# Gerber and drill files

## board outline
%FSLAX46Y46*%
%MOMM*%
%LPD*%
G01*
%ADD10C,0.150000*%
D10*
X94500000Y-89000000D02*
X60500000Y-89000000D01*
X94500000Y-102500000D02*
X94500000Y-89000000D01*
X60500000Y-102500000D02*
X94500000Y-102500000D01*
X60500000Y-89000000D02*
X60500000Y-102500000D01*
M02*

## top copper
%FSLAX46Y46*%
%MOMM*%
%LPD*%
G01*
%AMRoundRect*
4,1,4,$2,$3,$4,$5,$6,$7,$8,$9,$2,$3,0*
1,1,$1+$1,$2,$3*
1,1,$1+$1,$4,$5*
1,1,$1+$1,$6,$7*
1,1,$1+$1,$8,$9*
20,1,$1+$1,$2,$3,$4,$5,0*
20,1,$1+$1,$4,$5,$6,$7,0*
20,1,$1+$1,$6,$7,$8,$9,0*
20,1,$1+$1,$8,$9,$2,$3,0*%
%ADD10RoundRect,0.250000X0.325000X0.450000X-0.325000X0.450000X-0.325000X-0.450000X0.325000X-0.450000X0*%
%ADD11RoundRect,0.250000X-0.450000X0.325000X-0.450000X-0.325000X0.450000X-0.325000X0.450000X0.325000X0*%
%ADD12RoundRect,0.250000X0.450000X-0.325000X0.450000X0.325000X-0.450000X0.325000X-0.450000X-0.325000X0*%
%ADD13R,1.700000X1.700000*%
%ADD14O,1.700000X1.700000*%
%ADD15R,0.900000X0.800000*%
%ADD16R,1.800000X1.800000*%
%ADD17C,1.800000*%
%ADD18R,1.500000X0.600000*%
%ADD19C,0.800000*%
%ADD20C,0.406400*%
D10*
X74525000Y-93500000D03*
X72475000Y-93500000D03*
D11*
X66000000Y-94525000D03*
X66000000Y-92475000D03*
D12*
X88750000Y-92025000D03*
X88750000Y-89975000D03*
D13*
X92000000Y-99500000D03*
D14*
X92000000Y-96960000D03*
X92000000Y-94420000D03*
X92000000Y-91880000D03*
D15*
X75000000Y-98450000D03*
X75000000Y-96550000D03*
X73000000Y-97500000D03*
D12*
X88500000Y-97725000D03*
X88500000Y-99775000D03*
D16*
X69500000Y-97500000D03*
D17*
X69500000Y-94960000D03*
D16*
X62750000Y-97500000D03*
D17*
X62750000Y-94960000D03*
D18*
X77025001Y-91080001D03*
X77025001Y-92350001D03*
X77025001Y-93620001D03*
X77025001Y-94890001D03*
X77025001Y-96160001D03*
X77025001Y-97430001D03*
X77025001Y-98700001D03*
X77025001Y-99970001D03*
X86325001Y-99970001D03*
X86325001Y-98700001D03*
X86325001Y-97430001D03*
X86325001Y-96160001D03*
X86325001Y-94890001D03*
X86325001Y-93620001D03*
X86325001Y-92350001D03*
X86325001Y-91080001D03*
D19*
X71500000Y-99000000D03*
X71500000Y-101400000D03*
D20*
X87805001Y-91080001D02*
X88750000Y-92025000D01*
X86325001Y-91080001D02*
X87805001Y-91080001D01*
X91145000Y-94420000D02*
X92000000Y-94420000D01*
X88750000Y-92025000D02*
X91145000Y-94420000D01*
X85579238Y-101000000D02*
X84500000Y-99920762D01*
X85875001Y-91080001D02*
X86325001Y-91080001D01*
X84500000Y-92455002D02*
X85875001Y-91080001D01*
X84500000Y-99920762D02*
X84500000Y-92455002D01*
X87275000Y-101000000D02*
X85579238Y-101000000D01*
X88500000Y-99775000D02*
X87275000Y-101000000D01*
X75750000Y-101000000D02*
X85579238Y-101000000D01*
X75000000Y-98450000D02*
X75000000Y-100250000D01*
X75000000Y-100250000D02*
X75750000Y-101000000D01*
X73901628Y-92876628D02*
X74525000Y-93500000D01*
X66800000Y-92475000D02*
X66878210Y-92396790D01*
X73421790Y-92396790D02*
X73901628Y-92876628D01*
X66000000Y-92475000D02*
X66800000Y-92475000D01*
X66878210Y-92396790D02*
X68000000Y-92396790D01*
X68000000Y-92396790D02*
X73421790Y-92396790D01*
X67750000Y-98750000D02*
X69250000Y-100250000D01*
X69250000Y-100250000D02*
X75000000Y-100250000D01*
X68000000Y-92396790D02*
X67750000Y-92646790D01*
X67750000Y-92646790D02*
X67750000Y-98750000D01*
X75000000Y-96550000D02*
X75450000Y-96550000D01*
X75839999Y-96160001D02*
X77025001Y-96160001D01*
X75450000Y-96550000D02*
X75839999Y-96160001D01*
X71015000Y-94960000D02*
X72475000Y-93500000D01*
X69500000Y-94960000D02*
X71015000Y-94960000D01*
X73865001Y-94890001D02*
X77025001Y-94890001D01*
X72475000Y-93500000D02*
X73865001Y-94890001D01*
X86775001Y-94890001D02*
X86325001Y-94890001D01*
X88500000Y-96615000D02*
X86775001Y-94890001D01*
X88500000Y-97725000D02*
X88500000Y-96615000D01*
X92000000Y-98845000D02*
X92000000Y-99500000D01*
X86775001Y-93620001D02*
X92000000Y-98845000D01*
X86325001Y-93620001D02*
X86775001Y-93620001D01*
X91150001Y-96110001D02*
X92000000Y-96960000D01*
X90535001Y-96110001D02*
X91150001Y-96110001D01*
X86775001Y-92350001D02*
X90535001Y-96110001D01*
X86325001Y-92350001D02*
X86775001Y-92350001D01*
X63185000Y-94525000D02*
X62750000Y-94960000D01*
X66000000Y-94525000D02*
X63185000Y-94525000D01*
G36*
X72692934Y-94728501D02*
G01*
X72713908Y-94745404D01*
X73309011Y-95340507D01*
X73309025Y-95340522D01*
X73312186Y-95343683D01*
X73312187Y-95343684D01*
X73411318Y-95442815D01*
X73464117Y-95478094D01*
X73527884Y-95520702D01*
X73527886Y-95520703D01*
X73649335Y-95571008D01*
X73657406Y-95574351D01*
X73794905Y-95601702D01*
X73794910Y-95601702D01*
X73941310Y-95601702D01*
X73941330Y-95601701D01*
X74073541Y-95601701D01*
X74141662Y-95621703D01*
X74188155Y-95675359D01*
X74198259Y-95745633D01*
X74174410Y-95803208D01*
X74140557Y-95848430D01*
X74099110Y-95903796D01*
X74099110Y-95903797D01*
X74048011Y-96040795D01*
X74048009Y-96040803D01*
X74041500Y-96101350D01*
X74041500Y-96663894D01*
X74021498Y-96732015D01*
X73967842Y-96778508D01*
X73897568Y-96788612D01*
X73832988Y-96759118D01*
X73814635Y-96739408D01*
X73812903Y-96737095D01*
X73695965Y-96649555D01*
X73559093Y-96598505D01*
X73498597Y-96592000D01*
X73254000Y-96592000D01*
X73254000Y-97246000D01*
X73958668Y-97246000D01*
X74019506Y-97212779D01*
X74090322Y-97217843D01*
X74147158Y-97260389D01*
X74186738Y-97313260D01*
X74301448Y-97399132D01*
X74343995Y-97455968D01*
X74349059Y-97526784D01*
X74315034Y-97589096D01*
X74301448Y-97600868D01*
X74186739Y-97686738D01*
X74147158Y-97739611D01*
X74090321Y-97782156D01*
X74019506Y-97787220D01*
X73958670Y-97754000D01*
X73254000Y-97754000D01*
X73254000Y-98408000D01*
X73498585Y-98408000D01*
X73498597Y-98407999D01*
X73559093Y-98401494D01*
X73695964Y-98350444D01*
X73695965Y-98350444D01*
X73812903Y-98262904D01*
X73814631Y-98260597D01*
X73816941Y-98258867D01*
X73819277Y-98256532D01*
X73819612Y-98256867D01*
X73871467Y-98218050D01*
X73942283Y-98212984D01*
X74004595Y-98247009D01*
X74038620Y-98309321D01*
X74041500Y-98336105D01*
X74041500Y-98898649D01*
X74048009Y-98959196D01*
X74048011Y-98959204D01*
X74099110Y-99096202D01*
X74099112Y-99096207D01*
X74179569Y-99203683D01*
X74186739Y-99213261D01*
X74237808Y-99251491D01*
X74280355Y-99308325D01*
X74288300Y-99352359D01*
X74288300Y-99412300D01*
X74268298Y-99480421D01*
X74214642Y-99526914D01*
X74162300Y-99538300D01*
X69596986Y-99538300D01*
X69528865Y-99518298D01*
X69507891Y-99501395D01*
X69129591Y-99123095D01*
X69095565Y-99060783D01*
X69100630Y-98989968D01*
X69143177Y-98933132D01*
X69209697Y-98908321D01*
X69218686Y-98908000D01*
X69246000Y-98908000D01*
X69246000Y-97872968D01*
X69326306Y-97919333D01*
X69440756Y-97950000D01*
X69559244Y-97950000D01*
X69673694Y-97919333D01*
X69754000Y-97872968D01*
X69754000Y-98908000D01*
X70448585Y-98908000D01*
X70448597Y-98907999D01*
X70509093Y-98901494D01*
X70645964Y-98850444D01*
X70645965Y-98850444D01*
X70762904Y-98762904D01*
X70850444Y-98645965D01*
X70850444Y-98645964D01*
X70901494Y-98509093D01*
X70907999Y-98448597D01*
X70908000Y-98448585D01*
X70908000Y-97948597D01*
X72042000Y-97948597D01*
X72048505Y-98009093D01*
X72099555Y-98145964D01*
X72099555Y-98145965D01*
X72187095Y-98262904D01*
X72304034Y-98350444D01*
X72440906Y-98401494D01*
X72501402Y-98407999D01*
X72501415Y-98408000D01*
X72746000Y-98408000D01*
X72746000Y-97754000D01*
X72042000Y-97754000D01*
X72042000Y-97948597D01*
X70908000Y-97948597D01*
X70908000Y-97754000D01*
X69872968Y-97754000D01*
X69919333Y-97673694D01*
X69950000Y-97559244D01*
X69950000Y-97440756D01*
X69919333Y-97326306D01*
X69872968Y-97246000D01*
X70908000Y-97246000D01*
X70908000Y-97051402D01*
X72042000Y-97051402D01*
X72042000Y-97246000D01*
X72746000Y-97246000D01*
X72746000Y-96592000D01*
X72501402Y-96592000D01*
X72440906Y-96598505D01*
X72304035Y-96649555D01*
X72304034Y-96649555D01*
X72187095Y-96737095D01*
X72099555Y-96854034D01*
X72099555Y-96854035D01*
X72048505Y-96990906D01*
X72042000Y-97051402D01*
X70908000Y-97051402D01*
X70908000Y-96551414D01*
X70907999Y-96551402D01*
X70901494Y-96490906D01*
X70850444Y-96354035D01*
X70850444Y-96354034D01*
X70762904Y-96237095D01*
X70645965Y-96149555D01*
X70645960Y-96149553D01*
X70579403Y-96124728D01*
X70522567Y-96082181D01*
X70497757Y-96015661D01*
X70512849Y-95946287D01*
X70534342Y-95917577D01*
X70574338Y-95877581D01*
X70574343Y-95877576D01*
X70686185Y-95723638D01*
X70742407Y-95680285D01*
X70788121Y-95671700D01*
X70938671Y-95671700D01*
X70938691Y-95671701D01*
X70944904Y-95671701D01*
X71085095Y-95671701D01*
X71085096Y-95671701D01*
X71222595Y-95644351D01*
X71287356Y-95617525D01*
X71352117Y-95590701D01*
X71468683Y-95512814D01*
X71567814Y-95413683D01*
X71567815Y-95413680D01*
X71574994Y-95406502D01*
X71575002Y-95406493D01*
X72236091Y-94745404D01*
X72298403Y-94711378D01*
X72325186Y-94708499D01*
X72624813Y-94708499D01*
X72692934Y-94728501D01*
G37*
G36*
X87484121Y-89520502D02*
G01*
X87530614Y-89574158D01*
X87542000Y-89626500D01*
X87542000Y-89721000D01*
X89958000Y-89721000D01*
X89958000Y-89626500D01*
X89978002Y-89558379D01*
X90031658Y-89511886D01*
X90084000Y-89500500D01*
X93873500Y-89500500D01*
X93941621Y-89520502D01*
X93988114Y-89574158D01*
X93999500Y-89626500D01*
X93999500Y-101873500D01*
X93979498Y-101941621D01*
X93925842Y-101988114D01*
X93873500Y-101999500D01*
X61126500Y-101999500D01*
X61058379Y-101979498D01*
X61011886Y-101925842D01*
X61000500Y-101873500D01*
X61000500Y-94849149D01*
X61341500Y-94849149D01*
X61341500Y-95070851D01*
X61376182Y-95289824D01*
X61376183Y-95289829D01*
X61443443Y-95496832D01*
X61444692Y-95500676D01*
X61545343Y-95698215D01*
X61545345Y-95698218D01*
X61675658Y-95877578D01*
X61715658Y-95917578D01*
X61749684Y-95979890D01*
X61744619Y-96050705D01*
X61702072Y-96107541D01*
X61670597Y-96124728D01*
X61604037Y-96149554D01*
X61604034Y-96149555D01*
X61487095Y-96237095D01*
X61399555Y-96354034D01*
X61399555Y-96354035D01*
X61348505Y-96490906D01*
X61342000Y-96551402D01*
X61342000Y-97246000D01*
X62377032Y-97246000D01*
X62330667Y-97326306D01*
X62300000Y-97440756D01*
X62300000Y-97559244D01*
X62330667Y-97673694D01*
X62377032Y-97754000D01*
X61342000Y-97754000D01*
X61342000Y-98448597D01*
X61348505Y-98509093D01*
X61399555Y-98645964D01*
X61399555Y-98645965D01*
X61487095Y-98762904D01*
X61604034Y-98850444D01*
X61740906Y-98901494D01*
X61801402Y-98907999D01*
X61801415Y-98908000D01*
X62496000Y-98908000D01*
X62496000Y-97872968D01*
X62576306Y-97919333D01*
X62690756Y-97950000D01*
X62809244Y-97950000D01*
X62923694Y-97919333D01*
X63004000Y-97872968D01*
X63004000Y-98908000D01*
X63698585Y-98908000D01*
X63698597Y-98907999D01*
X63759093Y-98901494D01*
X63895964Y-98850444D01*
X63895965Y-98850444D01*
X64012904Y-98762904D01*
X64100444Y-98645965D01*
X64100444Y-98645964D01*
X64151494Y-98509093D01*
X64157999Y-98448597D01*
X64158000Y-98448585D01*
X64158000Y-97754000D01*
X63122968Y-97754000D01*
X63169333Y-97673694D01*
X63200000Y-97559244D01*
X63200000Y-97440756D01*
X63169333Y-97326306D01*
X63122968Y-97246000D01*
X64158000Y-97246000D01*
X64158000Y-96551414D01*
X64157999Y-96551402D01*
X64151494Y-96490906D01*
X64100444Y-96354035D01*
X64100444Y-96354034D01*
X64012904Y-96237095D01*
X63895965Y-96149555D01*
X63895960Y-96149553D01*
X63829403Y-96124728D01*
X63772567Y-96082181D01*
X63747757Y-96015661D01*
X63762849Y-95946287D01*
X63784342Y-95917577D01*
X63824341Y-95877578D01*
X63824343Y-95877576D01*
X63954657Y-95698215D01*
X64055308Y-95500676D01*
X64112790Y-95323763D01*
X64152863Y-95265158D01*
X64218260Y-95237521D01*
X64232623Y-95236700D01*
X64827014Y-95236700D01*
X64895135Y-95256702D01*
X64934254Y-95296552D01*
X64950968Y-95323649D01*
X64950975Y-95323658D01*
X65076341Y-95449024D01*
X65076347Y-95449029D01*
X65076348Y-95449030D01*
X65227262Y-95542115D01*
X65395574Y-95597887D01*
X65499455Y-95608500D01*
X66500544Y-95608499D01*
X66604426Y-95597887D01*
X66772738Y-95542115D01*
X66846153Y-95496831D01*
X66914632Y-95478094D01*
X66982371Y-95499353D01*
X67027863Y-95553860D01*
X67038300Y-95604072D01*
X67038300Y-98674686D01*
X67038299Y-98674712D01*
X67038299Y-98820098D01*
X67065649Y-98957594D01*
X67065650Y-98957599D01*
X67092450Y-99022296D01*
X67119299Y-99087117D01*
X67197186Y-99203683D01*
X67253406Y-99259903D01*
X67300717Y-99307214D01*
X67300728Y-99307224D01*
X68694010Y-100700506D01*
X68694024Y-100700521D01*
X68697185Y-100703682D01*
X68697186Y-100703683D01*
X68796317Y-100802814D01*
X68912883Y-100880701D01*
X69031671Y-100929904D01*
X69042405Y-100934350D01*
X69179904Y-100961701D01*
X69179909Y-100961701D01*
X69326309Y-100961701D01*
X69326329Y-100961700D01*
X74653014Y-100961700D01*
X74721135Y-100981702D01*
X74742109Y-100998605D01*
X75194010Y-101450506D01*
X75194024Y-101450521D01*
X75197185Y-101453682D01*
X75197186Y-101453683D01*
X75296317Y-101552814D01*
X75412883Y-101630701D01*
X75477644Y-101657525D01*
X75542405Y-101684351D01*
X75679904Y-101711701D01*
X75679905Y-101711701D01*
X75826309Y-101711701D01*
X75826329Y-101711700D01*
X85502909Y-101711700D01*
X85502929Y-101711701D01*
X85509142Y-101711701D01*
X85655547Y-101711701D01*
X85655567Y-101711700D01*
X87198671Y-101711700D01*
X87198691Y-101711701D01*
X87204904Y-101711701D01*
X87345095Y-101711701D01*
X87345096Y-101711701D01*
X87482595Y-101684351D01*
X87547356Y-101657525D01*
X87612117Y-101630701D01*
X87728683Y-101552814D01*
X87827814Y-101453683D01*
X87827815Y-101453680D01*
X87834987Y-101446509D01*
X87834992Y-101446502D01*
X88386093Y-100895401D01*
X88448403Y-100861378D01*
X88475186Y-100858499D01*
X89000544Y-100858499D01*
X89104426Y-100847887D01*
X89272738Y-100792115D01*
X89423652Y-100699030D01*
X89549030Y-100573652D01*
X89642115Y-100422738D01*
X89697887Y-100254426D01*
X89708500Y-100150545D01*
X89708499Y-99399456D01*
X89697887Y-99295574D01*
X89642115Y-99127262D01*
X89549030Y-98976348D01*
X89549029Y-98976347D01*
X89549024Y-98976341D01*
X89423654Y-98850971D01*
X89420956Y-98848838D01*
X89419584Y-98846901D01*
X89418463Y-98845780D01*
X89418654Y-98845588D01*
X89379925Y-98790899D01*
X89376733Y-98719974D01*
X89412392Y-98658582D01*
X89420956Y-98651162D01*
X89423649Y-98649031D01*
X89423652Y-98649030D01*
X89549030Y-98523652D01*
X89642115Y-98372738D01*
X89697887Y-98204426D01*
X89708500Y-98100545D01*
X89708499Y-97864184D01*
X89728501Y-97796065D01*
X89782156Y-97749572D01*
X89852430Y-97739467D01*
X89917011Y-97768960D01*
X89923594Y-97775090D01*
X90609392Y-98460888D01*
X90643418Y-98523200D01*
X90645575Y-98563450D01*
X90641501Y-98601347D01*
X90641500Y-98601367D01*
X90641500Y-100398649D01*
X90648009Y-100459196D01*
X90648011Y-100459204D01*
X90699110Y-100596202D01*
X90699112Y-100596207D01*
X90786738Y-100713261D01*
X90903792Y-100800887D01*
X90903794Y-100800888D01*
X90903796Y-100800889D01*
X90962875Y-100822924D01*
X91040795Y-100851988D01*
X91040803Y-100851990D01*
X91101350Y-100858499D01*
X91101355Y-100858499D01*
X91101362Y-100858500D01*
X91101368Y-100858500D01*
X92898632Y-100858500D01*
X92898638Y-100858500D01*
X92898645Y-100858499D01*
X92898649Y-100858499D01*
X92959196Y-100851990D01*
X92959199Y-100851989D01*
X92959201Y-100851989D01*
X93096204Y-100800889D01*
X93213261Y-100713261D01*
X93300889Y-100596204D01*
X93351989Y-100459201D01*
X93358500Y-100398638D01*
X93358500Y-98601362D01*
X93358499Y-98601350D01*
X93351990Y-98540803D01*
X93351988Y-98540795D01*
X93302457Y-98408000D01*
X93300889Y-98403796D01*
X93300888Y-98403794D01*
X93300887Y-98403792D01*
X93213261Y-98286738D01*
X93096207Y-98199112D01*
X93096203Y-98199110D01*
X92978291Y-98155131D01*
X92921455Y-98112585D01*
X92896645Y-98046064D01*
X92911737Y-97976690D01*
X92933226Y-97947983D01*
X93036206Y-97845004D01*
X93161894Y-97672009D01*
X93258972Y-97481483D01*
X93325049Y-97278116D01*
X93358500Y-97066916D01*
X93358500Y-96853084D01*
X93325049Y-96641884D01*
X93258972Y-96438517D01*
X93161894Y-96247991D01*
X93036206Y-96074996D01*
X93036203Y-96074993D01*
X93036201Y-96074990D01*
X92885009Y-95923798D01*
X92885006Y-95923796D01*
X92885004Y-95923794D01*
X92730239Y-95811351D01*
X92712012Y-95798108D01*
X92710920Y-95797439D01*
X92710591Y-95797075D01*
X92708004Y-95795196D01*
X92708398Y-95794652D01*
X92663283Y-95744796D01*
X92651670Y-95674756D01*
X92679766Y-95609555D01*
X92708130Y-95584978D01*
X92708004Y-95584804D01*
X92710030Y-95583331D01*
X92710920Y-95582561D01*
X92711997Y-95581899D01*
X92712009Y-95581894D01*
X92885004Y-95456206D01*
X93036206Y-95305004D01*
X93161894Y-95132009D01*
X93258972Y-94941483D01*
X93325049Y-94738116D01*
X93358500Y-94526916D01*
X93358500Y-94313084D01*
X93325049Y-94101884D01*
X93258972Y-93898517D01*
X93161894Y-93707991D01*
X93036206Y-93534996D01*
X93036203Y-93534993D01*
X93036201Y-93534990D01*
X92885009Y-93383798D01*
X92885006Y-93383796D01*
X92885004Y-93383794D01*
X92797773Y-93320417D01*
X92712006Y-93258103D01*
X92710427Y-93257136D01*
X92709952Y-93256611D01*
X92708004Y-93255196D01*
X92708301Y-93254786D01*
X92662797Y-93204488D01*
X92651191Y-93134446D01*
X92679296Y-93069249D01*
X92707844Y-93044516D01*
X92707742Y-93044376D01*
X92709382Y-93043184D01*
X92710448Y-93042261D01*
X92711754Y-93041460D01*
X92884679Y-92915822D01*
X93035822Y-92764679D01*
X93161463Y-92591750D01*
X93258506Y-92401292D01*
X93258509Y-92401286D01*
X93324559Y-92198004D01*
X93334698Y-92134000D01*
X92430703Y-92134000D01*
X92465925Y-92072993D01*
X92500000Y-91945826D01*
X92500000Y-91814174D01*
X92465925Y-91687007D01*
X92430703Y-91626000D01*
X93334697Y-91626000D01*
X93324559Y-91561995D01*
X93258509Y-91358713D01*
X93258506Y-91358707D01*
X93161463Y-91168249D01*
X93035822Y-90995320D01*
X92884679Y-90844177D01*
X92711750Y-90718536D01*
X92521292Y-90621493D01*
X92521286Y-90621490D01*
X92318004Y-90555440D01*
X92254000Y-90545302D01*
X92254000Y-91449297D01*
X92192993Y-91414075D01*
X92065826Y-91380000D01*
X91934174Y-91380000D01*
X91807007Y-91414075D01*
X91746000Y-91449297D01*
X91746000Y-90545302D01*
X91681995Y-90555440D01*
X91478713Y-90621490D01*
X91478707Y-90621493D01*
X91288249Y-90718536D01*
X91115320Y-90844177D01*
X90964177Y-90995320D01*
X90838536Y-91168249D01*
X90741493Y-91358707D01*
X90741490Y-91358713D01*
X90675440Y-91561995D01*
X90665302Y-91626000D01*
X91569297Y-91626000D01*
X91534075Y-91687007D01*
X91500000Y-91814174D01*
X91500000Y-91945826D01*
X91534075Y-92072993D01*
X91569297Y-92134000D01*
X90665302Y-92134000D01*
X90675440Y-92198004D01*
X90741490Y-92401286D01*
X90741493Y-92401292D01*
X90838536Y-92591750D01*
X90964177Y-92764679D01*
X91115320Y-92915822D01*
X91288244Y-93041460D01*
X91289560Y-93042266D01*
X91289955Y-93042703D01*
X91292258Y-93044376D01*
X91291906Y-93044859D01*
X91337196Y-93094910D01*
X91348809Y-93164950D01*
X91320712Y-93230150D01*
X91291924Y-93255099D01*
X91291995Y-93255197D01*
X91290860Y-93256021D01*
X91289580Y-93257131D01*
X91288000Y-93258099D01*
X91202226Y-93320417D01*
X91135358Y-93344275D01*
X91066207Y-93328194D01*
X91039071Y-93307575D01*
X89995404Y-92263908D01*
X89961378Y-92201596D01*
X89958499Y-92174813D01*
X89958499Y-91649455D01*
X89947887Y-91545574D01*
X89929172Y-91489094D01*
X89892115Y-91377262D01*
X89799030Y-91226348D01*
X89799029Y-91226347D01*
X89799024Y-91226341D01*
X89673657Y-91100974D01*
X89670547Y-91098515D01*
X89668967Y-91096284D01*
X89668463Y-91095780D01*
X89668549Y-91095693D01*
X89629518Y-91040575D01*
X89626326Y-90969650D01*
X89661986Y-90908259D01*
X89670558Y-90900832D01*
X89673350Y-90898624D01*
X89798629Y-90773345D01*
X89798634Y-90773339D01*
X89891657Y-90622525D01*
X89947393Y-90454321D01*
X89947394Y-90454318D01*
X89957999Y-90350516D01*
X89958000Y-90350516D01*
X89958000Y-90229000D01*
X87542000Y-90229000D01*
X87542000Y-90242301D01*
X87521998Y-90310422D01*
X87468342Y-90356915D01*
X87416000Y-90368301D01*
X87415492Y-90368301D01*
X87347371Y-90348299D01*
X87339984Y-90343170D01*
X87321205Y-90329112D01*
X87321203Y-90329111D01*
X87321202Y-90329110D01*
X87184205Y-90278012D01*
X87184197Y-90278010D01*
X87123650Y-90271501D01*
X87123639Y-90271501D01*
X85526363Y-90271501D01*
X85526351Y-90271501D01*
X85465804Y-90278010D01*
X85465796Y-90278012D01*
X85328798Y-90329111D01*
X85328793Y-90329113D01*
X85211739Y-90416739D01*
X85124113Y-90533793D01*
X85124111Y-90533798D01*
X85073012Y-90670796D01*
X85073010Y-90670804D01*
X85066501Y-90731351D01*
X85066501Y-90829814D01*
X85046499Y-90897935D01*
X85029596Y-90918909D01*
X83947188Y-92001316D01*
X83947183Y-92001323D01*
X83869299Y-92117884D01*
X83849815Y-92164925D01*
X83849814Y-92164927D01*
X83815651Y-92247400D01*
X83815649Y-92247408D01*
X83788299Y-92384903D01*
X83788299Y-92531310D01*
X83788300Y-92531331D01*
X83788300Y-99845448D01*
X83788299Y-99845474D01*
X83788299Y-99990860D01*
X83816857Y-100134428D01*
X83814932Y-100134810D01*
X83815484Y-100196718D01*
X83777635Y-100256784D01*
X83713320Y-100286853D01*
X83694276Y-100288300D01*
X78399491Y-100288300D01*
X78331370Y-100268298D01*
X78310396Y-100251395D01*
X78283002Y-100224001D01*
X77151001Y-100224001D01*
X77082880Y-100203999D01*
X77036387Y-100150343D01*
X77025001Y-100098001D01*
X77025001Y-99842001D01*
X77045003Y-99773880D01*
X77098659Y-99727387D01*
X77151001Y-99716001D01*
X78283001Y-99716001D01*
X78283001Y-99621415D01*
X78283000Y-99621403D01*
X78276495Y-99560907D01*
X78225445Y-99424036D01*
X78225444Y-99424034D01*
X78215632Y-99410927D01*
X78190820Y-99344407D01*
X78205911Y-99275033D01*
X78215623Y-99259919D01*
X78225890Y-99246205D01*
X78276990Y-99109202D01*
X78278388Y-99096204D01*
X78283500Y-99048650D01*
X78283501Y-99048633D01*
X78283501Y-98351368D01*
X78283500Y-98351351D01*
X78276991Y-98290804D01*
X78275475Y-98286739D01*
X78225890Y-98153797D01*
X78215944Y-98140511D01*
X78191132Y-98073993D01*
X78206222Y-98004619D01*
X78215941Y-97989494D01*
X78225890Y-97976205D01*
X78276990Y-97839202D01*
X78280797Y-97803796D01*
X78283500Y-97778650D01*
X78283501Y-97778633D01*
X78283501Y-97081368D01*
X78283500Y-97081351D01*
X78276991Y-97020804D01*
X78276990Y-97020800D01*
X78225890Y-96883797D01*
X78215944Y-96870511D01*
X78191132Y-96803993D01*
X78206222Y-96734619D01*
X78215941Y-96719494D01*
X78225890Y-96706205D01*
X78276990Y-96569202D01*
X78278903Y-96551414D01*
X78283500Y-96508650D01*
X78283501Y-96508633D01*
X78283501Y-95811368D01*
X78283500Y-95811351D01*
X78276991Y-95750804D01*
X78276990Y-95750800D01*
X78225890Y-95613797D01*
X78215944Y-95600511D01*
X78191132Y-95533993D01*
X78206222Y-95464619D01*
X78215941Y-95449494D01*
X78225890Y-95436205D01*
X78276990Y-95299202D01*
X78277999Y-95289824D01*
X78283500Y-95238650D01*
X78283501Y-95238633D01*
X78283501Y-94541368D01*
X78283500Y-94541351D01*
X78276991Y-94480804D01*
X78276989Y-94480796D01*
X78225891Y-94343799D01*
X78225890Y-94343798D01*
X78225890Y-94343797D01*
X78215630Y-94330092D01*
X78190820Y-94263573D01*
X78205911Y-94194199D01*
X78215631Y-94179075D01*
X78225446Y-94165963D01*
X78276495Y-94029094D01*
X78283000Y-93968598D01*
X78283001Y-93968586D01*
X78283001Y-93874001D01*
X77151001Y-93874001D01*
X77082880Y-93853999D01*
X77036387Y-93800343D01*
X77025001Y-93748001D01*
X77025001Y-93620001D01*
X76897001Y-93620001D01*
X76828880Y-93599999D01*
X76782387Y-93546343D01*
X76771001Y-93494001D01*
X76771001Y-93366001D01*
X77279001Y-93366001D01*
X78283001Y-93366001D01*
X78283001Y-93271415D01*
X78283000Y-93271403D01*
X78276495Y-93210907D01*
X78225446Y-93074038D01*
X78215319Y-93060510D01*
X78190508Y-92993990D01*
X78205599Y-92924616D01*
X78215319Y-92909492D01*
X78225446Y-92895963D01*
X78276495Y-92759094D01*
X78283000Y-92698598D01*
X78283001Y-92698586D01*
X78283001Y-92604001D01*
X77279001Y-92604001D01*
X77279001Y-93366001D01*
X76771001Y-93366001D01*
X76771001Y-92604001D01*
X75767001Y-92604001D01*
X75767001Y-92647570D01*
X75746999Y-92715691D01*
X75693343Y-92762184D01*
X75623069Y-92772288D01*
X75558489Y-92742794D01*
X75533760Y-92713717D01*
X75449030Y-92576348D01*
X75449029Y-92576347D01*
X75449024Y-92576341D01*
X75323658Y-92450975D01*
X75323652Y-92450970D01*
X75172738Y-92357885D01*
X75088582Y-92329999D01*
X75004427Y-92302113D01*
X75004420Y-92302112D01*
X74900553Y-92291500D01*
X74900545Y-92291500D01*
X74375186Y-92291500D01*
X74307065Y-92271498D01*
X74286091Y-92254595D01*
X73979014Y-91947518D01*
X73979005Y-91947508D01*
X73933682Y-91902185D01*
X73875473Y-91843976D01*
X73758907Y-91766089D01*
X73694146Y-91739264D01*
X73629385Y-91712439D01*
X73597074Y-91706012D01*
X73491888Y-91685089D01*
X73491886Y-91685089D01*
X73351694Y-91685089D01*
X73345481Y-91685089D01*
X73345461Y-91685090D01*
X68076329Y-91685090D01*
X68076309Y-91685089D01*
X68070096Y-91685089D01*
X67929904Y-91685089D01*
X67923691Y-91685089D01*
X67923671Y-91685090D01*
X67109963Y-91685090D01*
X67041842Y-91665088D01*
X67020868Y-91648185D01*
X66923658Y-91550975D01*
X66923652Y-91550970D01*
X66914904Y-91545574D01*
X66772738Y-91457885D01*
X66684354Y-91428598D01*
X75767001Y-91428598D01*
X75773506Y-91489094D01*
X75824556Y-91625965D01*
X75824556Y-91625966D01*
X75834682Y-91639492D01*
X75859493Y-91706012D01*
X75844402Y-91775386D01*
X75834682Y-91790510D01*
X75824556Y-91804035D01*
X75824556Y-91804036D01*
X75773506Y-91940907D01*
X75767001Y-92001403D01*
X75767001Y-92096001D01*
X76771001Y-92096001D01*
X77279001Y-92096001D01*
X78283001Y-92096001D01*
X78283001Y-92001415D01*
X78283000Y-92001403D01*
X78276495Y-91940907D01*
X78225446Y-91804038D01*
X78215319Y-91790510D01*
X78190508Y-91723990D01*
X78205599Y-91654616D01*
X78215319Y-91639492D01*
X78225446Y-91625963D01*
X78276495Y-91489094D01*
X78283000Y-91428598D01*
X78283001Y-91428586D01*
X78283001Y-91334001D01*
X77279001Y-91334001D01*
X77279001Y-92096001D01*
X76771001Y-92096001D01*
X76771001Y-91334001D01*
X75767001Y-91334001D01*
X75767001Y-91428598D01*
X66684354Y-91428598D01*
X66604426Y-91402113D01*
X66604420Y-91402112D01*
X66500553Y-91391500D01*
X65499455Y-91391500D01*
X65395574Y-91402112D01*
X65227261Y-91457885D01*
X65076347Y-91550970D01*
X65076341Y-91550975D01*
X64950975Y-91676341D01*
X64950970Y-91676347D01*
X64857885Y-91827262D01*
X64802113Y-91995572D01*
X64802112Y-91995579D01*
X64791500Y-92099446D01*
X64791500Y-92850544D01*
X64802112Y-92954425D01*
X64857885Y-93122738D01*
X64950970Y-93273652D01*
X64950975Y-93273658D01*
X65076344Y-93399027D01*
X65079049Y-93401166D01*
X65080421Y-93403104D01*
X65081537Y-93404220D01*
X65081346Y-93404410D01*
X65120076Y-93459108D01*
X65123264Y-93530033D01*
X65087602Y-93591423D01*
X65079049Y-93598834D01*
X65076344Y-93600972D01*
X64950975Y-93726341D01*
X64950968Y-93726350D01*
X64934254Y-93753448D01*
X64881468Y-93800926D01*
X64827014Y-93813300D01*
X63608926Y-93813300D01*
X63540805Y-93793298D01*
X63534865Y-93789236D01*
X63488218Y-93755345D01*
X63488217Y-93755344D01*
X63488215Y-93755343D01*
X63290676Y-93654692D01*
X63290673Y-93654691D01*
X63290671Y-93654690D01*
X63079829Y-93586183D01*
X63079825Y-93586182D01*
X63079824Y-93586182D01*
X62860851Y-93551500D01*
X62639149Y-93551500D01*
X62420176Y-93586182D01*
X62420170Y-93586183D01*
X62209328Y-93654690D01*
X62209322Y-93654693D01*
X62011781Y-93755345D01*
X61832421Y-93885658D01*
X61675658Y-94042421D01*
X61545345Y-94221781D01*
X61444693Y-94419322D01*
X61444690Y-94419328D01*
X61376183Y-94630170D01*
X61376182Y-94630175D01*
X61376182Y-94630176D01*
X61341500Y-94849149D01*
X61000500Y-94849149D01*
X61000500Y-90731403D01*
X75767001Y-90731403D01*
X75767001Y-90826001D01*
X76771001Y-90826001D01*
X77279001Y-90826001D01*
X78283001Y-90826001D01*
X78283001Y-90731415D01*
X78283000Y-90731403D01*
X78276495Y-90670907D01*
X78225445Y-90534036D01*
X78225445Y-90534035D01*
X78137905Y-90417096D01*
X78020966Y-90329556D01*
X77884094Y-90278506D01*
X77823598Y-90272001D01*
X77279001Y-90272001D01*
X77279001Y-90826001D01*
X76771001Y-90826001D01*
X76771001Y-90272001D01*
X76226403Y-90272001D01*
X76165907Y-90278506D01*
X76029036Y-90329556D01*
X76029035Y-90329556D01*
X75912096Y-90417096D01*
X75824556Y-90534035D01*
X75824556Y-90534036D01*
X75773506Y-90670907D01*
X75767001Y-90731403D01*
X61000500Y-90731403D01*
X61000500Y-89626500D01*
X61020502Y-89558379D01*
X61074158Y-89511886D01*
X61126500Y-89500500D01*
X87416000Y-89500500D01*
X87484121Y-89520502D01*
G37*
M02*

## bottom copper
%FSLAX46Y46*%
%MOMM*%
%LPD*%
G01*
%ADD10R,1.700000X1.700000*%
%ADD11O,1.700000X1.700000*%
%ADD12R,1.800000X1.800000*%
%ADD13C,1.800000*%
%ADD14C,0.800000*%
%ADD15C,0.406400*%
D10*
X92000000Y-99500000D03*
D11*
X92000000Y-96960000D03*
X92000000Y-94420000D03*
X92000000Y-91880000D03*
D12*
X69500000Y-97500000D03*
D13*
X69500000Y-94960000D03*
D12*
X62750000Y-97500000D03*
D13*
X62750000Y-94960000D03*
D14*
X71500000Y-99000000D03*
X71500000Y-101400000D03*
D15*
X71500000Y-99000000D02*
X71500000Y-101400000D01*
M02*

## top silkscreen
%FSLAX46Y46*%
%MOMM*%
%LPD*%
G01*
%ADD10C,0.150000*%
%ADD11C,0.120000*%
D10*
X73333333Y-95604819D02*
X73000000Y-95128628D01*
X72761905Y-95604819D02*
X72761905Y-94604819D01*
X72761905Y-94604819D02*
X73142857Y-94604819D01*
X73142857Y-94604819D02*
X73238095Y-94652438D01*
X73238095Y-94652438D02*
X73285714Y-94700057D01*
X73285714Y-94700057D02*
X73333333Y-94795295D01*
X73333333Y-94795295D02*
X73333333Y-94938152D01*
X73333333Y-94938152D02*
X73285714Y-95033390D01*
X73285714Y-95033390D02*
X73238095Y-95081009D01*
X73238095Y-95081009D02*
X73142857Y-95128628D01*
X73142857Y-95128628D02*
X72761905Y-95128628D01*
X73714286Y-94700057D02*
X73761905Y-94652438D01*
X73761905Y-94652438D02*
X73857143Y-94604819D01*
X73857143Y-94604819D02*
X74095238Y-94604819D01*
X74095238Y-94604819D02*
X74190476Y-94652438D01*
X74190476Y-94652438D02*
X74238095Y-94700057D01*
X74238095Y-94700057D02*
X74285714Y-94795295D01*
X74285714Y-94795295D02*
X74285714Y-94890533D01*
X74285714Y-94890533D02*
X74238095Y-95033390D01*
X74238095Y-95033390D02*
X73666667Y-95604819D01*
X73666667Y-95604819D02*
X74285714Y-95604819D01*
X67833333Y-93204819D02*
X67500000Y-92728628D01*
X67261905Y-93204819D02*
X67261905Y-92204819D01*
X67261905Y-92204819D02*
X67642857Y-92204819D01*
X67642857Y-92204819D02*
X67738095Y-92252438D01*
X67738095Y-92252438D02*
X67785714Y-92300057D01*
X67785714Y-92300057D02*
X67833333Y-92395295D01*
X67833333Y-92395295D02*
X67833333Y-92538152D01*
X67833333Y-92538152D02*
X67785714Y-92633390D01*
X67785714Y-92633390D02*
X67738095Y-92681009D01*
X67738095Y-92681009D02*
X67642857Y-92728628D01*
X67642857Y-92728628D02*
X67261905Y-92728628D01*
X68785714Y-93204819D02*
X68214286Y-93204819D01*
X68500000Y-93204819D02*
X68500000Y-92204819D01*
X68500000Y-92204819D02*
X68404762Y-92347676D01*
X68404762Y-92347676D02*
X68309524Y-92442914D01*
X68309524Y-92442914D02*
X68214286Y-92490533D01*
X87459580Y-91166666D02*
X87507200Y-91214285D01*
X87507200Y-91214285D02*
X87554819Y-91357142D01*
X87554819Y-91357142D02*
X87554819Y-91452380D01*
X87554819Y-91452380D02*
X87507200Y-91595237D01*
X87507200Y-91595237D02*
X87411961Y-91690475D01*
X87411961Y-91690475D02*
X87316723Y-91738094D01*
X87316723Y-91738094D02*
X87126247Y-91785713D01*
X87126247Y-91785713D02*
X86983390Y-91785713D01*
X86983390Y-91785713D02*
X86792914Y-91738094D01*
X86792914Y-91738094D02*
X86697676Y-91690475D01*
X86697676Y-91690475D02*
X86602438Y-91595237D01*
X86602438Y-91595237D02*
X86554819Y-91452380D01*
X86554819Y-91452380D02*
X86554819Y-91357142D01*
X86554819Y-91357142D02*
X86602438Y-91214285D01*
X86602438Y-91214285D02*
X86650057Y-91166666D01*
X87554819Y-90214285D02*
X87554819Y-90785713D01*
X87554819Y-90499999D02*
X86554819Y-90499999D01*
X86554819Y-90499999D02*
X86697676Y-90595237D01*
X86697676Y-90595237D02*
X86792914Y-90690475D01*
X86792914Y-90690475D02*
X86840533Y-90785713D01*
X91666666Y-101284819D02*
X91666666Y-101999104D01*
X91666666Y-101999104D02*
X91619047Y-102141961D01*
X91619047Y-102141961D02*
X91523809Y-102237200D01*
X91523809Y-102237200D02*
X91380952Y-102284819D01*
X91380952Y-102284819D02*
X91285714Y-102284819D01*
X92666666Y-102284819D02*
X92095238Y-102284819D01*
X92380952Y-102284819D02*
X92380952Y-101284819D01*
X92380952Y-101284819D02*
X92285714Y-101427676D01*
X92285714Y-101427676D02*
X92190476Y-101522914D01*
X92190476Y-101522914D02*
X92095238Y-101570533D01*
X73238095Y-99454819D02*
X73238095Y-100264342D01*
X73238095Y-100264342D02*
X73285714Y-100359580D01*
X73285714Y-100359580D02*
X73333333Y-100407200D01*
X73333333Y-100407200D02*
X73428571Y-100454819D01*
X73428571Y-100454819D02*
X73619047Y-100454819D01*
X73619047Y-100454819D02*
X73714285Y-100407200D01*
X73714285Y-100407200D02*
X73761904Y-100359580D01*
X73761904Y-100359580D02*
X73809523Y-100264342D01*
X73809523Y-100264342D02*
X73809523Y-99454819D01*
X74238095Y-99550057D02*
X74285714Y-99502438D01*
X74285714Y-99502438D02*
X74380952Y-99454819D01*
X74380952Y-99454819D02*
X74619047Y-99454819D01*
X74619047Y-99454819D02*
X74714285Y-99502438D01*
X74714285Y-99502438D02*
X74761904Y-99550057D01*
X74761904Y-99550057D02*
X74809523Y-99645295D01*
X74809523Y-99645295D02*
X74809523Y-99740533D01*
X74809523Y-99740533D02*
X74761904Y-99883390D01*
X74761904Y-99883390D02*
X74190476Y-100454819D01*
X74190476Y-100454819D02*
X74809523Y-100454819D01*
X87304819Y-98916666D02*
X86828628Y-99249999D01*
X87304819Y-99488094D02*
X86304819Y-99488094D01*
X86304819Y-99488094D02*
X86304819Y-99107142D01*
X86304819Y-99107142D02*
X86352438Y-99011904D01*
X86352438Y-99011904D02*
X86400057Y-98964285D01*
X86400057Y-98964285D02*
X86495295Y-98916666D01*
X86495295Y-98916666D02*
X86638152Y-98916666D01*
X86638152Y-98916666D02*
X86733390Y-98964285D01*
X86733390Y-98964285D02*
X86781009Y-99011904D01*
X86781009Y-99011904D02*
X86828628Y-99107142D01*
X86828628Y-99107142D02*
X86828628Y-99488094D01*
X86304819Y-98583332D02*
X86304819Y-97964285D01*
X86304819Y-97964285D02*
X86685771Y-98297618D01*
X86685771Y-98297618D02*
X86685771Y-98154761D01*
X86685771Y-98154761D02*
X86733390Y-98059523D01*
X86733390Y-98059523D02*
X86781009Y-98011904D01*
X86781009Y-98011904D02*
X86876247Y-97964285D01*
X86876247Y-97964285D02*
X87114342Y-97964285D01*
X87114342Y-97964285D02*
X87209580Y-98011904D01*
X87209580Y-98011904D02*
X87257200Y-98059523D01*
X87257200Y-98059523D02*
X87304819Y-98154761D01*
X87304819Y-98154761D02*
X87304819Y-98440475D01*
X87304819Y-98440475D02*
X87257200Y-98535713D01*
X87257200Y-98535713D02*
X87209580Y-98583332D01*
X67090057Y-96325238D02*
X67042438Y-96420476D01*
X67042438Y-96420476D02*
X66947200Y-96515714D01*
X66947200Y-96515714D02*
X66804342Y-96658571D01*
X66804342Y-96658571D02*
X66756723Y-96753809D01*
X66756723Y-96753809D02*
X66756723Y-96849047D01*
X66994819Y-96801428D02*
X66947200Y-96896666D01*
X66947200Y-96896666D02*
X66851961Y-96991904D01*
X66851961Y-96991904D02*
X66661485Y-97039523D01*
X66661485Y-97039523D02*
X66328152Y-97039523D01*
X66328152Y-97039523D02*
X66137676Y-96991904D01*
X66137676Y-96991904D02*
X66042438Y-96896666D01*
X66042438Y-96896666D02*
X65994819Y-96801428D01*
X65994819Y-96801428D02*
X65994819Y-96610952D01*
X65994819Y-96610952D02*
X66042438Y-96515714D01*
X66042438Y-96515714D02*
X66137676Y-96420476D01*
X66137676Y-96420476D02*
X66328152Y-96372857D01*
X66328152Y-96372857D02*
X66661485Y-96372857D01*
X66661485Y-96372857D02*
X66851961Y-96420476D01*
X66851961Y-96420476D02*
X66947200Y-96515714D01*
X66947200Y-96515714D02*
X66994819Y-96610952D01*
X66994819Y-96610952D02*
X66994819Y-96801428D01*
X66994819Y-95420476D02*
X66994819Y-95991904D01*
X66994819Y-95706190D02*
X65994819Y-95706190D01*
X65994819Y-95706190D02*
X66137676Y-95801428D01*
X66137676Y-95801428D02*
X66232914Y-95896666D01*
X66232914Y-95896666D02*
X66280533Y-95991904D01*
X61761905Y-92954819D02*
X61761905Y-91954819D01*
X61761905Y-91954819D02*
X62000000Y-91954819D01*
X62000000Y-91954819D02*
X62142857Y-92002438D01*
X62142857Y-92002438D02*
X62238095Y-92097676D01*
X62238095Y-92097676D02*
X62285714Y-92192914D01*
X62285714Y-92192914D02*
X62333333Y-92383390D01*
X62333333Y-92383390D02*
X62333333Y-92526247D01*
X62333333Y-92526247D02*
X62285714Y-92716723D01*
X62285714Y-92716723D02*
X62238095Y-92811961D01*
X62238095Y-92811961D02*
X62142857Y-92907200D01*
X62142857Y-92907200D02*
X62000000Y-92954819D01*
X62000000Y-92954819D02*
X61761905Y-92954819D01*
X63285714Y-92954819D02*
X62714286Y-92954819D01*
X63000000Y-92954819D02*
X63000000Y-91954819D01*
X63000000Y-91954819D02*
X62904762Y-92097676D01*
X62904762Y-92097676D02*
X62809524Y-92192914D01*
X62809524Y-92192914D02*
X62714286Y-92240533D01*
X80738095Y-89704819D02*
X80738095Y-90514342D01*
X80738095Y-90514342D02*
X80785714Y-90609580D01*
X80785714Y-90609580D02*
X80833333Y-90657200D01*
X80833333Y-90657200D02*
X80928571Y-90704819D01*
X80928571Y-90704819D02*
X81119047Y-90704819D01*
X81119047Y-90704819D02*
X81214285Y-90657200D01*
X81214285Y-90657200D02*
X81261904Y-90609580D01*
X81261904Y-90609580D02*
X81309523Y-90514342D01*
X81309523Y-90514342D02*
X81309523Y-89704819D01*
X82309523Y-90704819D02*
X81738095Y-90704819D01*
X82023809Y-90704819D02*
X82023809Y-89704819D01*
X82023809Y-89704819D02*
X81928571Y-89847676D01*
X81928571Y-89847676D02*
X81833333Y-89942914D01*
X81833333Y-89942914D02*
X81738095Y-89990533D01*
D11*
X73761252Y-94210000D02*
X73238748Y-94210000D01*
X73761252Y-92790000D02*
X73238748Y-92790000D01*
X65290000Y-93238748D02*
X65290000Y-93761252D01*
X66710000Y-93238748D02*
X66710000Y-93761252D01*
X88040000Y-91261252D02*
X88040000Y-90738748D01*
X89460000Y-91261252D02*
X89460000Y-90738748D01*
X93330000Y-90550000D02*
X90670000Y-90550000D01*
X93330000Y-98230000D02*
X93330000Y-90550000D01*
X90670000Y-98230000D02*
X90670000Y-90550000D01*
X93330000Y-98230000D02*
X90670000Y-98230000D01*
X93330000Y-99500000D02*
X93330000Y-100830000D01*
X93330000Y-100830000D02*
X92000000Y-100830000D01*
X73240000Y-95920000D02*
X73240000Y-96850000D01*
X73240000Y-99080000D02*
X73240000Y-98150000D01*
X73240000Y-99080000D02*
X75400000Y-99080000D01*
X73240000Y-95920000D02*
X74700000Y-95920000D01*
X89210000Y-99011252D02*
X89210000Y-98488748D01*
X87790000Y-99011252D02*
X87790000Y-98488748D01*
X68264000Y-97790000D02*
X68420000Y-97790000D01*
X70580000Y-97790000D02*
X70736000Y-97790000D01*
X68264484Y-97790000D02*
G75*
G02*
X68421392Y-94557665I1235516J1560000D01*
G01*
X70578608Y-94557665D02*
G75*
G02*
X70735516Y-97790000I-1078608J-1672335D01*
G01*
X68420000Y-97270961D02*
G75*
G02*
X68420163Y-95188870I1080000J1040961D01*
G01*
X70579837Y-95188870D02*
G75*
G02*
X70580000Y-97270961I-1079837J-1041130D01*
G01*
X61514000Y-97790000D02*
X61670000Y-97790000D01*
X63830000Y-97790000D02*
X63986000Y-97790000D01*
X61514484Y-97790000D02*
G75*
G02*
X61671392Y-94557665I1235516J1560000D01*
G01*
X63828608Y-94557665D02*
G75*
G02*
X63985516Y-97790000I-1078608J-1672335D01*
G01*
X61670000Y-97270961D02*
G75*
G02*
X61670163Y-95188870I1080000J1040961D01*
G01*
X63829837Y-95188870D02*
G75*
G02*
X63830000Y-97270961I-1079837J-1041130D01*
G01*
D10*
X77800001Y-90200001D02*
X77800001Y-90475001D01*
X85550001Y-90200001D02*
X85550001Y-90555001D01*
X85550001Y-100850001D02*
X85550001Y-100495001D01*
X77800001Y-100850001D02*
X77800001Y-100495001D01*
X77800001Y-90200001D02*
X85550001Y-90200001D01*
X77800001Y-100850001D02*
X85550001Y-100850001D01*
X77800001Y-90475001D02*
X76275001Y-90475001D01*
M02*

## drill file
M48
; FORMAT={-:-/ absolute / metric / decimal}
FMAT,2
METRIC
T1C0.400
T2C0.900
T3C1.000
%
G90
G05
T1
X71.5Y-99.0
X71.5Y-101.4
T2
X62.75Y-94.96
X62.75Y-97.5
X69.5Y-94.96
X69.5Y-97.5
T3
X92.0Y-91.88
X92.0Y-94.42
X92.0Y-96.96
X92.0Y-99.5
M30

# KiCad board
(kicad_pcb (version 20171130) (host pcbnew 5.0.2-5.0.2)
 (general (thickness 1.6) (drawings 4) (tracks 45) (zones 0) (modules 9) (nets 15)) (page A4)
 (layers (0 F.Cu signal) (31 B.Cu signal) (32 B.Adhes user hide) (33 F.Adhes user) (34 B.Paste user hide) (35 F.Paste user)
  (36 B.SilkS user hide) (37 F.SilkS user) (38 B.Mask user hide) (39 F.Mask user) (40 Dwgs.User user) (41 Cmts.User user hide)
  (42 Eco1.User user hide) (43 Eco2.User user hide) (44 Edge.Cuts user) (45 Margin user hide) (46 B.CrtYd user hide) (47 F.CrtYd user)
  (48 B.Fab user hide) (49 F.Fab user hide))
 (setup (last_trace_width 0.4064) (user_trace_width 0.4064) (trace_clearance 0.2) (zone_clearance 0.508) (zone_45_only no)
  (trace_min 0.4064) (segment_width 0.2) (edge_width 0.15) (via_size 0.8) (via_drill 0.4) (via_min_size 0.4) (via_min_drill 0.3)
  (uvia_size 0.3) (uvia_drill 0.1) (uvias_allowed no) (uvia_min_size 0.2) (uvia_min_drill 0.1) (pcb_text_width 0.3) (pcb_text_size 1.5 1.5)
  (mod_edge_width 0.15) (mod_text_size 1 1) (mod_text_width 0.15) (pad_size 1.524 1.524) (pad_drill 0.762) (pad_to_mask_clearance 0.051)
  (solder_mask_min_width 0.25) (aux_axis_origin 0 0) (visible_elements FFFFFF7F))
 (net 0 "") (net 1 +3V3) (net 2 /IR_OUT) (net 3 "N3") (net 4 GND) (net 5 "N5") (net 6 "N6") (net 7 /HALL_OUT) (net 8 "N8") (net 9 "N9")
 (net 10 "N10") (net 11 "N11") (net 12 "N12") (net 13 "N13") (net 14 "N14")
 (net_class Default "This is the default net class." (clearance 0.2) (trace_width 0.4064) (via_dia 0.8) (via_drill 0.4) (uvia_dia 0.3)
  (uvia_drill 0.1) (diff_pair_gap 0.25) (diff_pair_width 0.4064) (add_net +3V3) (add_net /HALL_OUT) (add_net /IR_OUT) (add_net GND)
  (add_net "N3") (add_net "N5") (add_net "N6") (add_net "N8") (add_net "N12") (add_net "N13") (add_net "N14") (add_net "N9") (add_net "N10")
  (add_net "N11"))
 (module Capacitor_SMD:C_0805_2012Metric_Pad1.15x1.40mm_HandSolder (layer F.Cu) (at 73.5 93.5 180)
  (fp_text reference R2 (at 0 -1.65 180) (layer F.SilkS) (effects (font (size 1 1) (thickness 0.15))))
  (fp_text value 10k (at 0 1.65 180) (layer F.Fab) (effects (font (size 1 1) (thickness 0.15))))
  (fp_line (start -0.261252 -0.71) (end 0.261252 -0.71) (layer F.SilkS) (width 0.12))
  (fp_line (start -0.261252 0.71) (end 0.261252 0.71) (layer F.SilkS) (width 0.12))
  (pad 1 smd roundrect (at -1.025 0 180) (size 1.15 1.4) (layers F.Cu F.Paste F.Mask) (roundrect_rratio 0.217391) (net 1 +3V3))
  (pad 2 smd roundrect (at 1.025 0 180) (size 1.15 1.4) (layers F.Cu F.Paste F.Mask) (roundrect_rratio 0.217391) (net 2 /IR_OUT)))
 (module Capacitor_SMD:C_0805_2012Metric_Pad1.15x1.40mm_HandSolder (layer F.Cu) (at 66 93.5 270)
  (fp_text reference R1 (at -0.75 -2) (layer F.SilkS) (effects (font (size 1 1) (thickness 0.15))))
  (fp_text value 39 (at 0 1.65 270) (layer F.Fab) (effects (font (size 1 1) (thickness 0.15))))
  (fp_line (start -0.261252 0.71) (end 0.261252 0.71) (layer F.SilkS) (width 0.12))
  (fp_line (start -0.261252 -0.71) (end 0.261252 -0.71) (layer F.SilkS) (width 0.12))
  (pad 2 smd roundrect (at 1.025 0 270) (size 1.15 1.4) (layers F.Cu F.Paste F.Mask) (roundrect_rratio 0.217391) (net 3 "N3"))
  (pad 1 smd roundrect (at -1.025 0 270) (size 1.15 1.4) (layers F.Cu F.Paste F.Mask) (roundrect_rratio 0.217391) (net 1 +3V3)))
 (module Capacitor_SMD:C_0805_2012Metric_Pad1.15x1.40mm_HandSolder (layer F.Cu) (at 88.75 91 90)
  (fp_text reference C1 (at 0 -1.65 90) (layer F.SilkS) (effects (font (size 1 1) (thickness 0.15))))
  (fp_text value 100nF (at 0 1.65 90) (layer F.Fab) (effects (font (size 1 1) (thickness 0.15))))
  (fp_line (start -0.261252 -0.71) (end 0.261252 -0.71) (layer F.SilkS) (width 0.12))
  (fp_line (start -0.261252 0.71) (end 0.261252 0.71) (layer F.SilkS) (width 0.12))
  (pad 1 smd roundrect (at -1.025 0 90) (size 1.15 1.4) (layers F.Cu F.Paste F.Mask) (roundrect_rratio 0.217391) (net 1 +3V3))
  (pad 2 smd roundrect (at 1.025 0 90) (size 1.15 1.4) (layers F.Cu F.Paste F.Mask) (roundrect_rratio 0.217391) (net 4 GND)))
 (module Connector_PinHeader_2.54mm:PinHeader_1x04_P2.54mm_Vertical (layer F.Cu) (at 92 99.5 180)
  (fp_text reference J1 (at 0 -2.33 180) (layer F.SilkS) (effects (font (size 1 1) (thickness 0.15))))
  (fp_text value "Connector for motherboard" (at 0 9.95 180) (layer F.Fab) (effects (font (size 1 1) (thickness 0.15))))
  (fp_line (start -1.33 8.95) (end 1.33 8.95) (layer F.SilkS) (width 0.12))
  (fp_line (start -1.33 1.27) (end -1.33 8.95) (layer F.SilkS) (width 0.12))
  (fp_line (start 1.33 1.27) (end 1.33 8.95) (layer F.SilkS) (width 0.12))
  (fp_line (start -1.33 1.27) (end 1.33 1.27) (layer F.SilkS) (width 0.12))
  (fp_line (start -1.33 0) (end -1.33 -1.33) (layer F.SilkS) (width 0.12))
  (fp_line (start -1.33 -1.33) (end 0 -1.33) (layer F.SilkS) (width 0.12))
  (pad 1 thru_hole rect (at 0 0 180) (size 1.7 1.7) (drill 1) (layers *.Cu *.Mask) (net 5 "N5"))
  (pad 2 thru_hole oval (at 0 2.54 180) (size 1.7 1.7) (drill 1) (layers *.Cu *.Mask) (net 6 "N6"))
  (pad 3 thru_hole oval (at 0 5.08 180) (size 1.7 1.7) (drill 1) (layers *.Cu *.Mask) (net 1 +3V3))
  (pad 4 thru_hole oval (at 0 7.62 180) (size 1.7 1.7) (drill 1) (layers *.Cu *.Mask) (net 4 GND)))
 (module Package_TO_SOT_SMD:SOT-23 (layer F.Cu) (at 74 97.5 180)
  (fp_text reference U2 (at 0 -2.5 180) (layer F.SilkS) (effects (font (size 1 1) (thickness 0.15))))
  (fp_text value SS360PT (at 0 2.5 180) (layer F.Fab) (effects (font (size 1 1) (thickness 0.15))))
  (fp_line (start 0.76 1.58) (end 0.76 0.65) (layer F.SilkS) (width 0.12))
  (fp_line (start 0.76 -1.58) (end 0.76 -0.65) (layer F.SilkS) (width 0.12))
  (fp_line (start 0.76 -1.58) (end -1.4 -1.58) (layer F.SilkS) (width 0.12))
  (fp_line (start 0.76 1.58) (end -0.7 1.58) (layer F.SilkS) (width 0.12))
  (pad 1 smd rect (at -1 -0.95 180) (size 0.9 0.8) (layers F.Cu F.Paste F.Mask) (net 1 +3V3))
  (pad 2 smd rect (at -1 0.95 180) (size 0.9 0.8) (layers F.Cu F.Paste F.Mask) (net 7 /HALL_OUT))
  (pad 3 smd rect (at 1 0 180) (size 0.9 0.8) (layers F.Cu F.Paste F.Mask) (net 4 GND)))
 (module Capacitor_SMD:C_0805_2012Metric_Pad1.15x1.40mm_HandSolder (layer F.Cu) (at 88.5 98.75 90)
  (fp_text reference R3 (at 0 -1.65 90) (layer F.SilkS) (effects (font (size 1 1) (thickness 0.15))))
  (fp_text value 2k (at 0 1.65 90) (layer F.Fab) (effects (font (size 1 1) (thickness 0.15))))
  (fp_line (start -0.261252 0.71) (end 0.261252 0.71) (layer F.SilkS) (width 0.12))
  (fp_line (start -0.261252 -0.71) (end 0.261252 -0.71) (layer F.SilkS) (width 0.12))
  (pad 2 smd roundrect (at 1.025 0 90) (size 1.15 1.4) (layers F.Cu F.Paste F.Mask) (roundrect_rratio 0.217391) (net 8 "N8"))
  (pad 1 smd roundrect (at -1.025 0 90) (size 1.15 1.4) (layers F.Cu F.Paste F.Mask) (roundrect_rratio 0.217391) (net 1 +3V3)))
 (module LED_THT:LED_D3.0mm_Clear (layer F.Cu) (at 69.5 97.5 90)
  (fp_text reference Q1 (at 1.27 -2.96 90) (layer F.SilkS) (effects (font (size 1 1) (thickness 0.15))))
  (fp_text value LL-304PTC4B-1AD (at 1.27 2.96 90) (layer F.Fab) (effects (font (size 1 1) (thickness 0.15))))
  (fp_line (start -0.29 -1.236) (end -0.29 -1.08) (layer F.SilkS) (width 0.12))
  (fp_line (start -0.29 1.08) (end -0.29 1.236) (layer F.SilkS) (width 0.12))
  (fp_arc (start 1.27 0) (end -0.29 -1.235516) (angle 108.8) (layer F.SilkS) (width 0.12))
  (fp_arc (start 1.27 0) (end -0.29 1.235516) (angle -108.8) (layer F.SilkS) (width 0.12))
  (fp_arc (start 1.27 0) (end 0.229039 -1.08) (angle 87.9) (layer F.SilkS) (width 0.12))
  (fp_arc (start 1.27 0) (end 0.229039 1.08) (angle -87.9) (layer F.SilkS) (width 0.12))
  (pad 1 thru_hole rect (at 0 0 90) (size 1.8 1.8) (drill 0.9) (layers *.Cu *.Mask) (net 4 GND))
  (pad 2 thru_hole circle (at 2.54 0 90) (size 1.8 1.8) (drill 0.9) (layers *.Cu *.Mask) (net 2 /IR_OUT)))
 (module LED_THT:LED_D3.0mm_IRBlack (layer F.Cu) (at 62.75 97.5 90)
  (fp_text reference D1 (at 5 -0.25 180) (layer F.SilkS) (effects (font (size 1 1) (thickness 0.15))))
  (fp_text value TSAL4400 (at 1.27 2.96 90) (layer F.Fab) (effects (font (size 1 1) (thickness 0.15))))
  (fp_line (start -0.29 -1.236) (end -0.29 -1.08) (layer F.SilkS) (width 0.12))
  (fp_line (start -0.29 1.08) (end -0.29 1.236) (layer F.SilkS) (width 0.12))
  (fp_arc (start 1.27 0) (end -0.29 -1.235516) (angle 108.8) (layer F.SilkS) (width 0.12))
  (fp_arc (start 1.27 0) (end -0.29 1.235516) (angle -108.8) (layer F.SilkS) (width 0.12))
  (fp_arc (start 1.27 0) (end 0.229039 -1.08) (angle 87.9) (layer F.SilkS) (width 0.12))
  (fp_arc (start 1.27 0) (end 0.229039 1.08) (angle -87.9) (layer F.SilkS) (width 0.12))
  (pad 1 thru_hole rect (at 0 0 90) (size 1.8 1.8) (drill 0.9) (layers *.Cu *.Mask) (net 4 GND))
  (pad 2 thru_hole circle (at 2.54 0 90) (size 1.8 1.8) (drill 0.9) (layers *.Cu *.Mask) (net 3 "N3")))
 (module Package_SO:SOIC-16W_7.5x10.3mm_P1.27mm (layer F.Cu) (at 81.675001 95.525001)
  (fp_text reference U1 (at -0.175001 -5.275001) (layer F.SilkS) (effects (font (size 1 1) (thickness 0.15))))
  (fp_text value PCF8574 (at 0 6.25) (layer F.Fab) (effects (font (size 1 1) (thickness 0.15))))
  (fp_line (start -3.875 -5.325) (end -3.875 -5.05) (layer F.SilkS) (width 0.15))
  (fp_line (start 3.875 -5.325) (end 3.875 -4.97) (layer F.SilkS) (width 0.15))
  (fp_line (start 3.875 5.325) (end 3.875 4.97) (layer F.SilkS) (width 0.15))
  (fp_line (start -3.875 5.325) (end -3.875 4.97) (layer F.SilkS) (width 0.15))
  (fp_line (start -3.875 -5.325) (end 3.875 -5.325) (layer F.SilkS) (width 0.15))
  (fp_line (start -3.875 5.325) (end 3.875 5.325) (layer F.SilkS) (width 0.15))
  (fp_line (start -3.875 -5.05) (end -5.4 -5.05) (layer F.SilkS) (width 0.15))
  (pad 1 smd rect (at -4.65 -4.445) (size 1.5 0.6) (layers F.Cu F.Paste F.Mask) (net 4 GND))
  (pad 2 smd rect (at -4.65 -3.175) (size 1.5 0.6) (layers F.Cu F.Paste F.Mask) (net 4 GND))
  (pad 3 smd rect (at -4.65 -1.905) (size 1.5 0.6) (layers F.Cu F.Paste F.Mask) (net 4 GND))
  (pad 4 smd rect (at -4.65 -0.635) (size 1.5 0.6) (layers F.Cu F.Paste F.Mask) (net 2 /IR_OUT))
  (pad 5 smd rect (at -4.65 0.635) (size 1.5 0.6) (layers F.Cu F.Paste F.Mask) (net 7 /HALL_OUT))
  (pad 6 smd rect (at -4.65 1.905) (size 1.5 0.6) (layers F.Cu F.Paste F.Mask) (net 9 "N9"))
  (pad 7 smd rect (at -4.65 3.175) (size 1.5 0.6) (layers F.Cu F.Paste F.Mask) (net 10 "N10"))
  (pad 8 smd rect (at -4.65 4.445) (size 1.5 0.6) (layers F.Cu F.Paste F.Mask) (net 4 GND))
  (pad 9 smd rect (at 4.65 4.445) (size 1.5 0.6) (layers F.Cu F.Paste F.Mask) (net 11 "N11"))
  (pad 10 smd rect (at 4.65 3.175) (size 1.5 0.6) (layers F.Cu F.Paste F.Mask) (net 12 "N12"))
  (pad 11 smd rect (at 4.65 1.905) (size 1.5 0.6) (layers F.Cu F.Paste F.Mask) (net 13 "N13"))
  (pad 12 smd rect (at 4.65 0.635) (size 1.5 0.6) (layers F.Cu F.Paste F.Mask) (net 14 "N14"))
  (pad 13 smd rect (at 4.65 -0.635) (size 1.5 0.6) (layers F.Cu F.Paste F.Mask) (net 8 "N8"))
  (pad 14 smd rect (at 4.65 -1.905) (size 1.5 0.6) (layers F.Cu F.Paste F.Mask) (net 5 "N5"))
  (pad 15 smd rect (at 4.65 -3.175) (size 1.5 0.6) (layers F.Cu F.Paste F.Mask) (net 6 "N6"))
  (pad 16 smd rect (at 4.65 -4.445) (size 1.5 0.6) (layers F.Cu F.Paste F.Mask) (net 1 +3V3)))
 (gr_line (start 94.5 89) (end 60.5 89) (layer Edge.Cuts) (width 0.15))
 (gr_line (start 94.5 102.5) (end 94.5 89) (layer Edge.Cuts) (width 0.15))
 (gr_line (start 60.5 102.5) (end 94.5 102.5) (layer Edge.Cuts) (width 0.15))
 (gr_line (start 60.5 89) (end 60.5 102.5) (layer Edge.Cuts) (width 0.15))
 (segment (start 87.805001 91.080001) (end 88.75 92.025) (width 0.4064) (layer F.Cu) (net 1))
 (segment (start 86.325001 91.080001) (end 87.805001 91.080001) (width 0.4064) (layer F.Cu) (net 1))
 (segment (start 91.145 94.42) (end 92 94.42) (width 0.4064) (layer F.Cu) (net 1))
 (segment (start 88.75 92.025) (end 91.145 94.42) (width 0.4064) (layer F.Cu) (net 1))
 (segment (start 85.579238 101) (end 84.5 99.920762) (width 0.4064) (layer F.Cu) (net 1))
 (segment (start 85.875001 91.080001) (end 86.325001 91.080001) (width 0.4064) (layer F.Cu) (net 1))
 (segment (start 84.5 92.455002) (end 85.875001 91.080001) (width 0.4064) (layer F.Cu) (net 1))
 (segment (start 84.5 99.920762) (end 84.5 92.455002) (width 0.4064) (layer F.Cu) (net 1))
 (segment (start 87.275 101) (end 85.579238 101) (width 0.4064) (layer F.Cu) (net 1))
 (segment (start 88.5 99.775) (end 87.275 101) (width 0.4064) (layer F.Cu) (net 1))
 (segment (start 75.75 101) (end 85.579238 101) (width 0.4064) (layer F.Cu) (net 1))
 (segment (start 75 98.45) (end 75 100.25) (width 0.4064) (layer F.Cu) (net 1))
 (segment (start 75 100.25) (end 75.75 101) (width 0.4064) (layer F.Cu) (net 1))
 (segment (start 73.901628 92.876628) (end 74.525 93.5) (width 0.4064) (layer F.Cu) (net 1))
 (segment (start 66.8 92.475) (end 66.87821 92.39679) (width 0.4064) (layer F.Cu) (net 1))
 (segment (start 73.42179 92.39679) (end 73.901628 92.876628) (width 0.4064) (layer F.Cu) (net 1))
 (segment (start 66 92.475) (end 66.8 92.475) (width 0.4064) (layer F.Cu) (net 1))
 (segment (start 66.87821 92.39679) (end 68 92.39679) (width 0.4064) (layer F.Cu) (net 1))
 (segment (start 68 92.39679) (end 73.42179 92.39679) (width 0.4064) (layer F.Cu) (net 1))
 (segment (start 67.75 98.75) (end 69.25 100.25) (width 0.4064) (layer F.Cu) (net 1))
 (segment (start 69.25 100.25) (end 75 100.25) (width 0.4064) (layer F.Cu) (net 1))
 (segment (start 68 92.39679) (end 67.75 92.64679) (width 0.4064) (layer F.Cu) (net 1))
 (segment (start 67.75 92.64679) (end 67.75 98.75) (width 0.4064) (layer F.Cu) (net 1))
 (segment (start 75 96.55) (end 75.45 96.55) (width 0.4064) (layer F.Cu) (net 7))
 (segment (start 75.839999 96.160001) (end 77.025001 96.160001) (width 0.4064) (layer F.Cu) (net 7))
 (segment (start 75.45 96.55) (end 75.839999 96.160001) (width 0.4064) (layer F.Cu) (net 7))
 (via (at 71.5 99) (size 0.8) (drill 0.4) (layers F.Cu B.Cu) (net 4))
 (via (at 71.5 101.4) (size 0.8) (drill 0.4) (layers F.Cu B.Cu) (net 4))
 (segment (start 71.5 99) (end 71.5 101.4) (width 0.4064) (layer B.Cu) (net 4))
 (segment (start 71.015 94.96) (end 72.475 93.5) (width 0.4064) (layer F.Cu) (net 2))
 (segment (start 69.5 94.96) (end 71.015 94.96) (width 0.4064) (layer F.Cu) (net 2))
 (segment (start 73.865001 94.890001) (end 77.025001 94.890001) (width 0.4064) (layer F.Cu) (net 2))
 (segment (start 72.475 93.5) (end 73.865001 94.890001) (width 0.4064) (layer F.Cu) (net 2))
 (segment (start 86.775001 94.890001) (end 86.325001 94.890001) (width 0.4064) (layer F.Cu) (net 8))
 (segment (start 88.5 96.615) (end 86.775001 94.890001) (width 0.4064) (layer F.Cu) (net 8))
 (segment (start 88.5 97.725) (end 88.5 96.615) (width 0.4064) (layer F.Cu) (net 8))
 (segment (start 92 98.845) (end 92 99.5) (width 0.4064) (layer F.Cu) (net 5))
 (segment (start 86.775001 93.620001) (end 92 98.845) (width 0.4064) (layer F.Cu) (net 5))
 (segment (start 86.325001 93.620001) (end 86.775001 93.620001) (width 0.4064) (layer F.Cu) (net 5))
 (segment (start 91.150001 96.110001) (end 92 96.96) (width 0.4064) (layer F.Cu) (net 6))
 (segment (start 90.535001 96.110001) (end 91.150001 96.110001) (width 0.4064) (layer F.Cu) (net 6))
 (segment (start 86.775001 92.350001) (end 90.535001 96.110001) (width 0.4064) (layer F.Cu) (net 6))
 (segment (start 86.325001 92.350001) (end 86.775001 92.350001) (width 0.4064) (layer F.Cu) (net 6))
 (segment (start 63.185 94.525) (end 62.75 94.96) (width 0.4064) (layer F.Cu) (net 3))
 (segment (start 66 94.525) (end 63.185 94.525) (width 0.4064) (layer F.Cu) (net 3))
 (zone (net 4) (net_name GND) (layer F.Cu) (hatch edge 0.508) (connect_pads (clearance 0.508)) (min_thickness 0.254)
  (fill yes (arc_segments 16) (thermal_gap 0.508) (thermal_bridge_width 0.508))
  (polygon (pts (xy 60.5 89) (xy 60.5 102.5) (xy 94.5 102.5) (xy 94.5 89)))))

